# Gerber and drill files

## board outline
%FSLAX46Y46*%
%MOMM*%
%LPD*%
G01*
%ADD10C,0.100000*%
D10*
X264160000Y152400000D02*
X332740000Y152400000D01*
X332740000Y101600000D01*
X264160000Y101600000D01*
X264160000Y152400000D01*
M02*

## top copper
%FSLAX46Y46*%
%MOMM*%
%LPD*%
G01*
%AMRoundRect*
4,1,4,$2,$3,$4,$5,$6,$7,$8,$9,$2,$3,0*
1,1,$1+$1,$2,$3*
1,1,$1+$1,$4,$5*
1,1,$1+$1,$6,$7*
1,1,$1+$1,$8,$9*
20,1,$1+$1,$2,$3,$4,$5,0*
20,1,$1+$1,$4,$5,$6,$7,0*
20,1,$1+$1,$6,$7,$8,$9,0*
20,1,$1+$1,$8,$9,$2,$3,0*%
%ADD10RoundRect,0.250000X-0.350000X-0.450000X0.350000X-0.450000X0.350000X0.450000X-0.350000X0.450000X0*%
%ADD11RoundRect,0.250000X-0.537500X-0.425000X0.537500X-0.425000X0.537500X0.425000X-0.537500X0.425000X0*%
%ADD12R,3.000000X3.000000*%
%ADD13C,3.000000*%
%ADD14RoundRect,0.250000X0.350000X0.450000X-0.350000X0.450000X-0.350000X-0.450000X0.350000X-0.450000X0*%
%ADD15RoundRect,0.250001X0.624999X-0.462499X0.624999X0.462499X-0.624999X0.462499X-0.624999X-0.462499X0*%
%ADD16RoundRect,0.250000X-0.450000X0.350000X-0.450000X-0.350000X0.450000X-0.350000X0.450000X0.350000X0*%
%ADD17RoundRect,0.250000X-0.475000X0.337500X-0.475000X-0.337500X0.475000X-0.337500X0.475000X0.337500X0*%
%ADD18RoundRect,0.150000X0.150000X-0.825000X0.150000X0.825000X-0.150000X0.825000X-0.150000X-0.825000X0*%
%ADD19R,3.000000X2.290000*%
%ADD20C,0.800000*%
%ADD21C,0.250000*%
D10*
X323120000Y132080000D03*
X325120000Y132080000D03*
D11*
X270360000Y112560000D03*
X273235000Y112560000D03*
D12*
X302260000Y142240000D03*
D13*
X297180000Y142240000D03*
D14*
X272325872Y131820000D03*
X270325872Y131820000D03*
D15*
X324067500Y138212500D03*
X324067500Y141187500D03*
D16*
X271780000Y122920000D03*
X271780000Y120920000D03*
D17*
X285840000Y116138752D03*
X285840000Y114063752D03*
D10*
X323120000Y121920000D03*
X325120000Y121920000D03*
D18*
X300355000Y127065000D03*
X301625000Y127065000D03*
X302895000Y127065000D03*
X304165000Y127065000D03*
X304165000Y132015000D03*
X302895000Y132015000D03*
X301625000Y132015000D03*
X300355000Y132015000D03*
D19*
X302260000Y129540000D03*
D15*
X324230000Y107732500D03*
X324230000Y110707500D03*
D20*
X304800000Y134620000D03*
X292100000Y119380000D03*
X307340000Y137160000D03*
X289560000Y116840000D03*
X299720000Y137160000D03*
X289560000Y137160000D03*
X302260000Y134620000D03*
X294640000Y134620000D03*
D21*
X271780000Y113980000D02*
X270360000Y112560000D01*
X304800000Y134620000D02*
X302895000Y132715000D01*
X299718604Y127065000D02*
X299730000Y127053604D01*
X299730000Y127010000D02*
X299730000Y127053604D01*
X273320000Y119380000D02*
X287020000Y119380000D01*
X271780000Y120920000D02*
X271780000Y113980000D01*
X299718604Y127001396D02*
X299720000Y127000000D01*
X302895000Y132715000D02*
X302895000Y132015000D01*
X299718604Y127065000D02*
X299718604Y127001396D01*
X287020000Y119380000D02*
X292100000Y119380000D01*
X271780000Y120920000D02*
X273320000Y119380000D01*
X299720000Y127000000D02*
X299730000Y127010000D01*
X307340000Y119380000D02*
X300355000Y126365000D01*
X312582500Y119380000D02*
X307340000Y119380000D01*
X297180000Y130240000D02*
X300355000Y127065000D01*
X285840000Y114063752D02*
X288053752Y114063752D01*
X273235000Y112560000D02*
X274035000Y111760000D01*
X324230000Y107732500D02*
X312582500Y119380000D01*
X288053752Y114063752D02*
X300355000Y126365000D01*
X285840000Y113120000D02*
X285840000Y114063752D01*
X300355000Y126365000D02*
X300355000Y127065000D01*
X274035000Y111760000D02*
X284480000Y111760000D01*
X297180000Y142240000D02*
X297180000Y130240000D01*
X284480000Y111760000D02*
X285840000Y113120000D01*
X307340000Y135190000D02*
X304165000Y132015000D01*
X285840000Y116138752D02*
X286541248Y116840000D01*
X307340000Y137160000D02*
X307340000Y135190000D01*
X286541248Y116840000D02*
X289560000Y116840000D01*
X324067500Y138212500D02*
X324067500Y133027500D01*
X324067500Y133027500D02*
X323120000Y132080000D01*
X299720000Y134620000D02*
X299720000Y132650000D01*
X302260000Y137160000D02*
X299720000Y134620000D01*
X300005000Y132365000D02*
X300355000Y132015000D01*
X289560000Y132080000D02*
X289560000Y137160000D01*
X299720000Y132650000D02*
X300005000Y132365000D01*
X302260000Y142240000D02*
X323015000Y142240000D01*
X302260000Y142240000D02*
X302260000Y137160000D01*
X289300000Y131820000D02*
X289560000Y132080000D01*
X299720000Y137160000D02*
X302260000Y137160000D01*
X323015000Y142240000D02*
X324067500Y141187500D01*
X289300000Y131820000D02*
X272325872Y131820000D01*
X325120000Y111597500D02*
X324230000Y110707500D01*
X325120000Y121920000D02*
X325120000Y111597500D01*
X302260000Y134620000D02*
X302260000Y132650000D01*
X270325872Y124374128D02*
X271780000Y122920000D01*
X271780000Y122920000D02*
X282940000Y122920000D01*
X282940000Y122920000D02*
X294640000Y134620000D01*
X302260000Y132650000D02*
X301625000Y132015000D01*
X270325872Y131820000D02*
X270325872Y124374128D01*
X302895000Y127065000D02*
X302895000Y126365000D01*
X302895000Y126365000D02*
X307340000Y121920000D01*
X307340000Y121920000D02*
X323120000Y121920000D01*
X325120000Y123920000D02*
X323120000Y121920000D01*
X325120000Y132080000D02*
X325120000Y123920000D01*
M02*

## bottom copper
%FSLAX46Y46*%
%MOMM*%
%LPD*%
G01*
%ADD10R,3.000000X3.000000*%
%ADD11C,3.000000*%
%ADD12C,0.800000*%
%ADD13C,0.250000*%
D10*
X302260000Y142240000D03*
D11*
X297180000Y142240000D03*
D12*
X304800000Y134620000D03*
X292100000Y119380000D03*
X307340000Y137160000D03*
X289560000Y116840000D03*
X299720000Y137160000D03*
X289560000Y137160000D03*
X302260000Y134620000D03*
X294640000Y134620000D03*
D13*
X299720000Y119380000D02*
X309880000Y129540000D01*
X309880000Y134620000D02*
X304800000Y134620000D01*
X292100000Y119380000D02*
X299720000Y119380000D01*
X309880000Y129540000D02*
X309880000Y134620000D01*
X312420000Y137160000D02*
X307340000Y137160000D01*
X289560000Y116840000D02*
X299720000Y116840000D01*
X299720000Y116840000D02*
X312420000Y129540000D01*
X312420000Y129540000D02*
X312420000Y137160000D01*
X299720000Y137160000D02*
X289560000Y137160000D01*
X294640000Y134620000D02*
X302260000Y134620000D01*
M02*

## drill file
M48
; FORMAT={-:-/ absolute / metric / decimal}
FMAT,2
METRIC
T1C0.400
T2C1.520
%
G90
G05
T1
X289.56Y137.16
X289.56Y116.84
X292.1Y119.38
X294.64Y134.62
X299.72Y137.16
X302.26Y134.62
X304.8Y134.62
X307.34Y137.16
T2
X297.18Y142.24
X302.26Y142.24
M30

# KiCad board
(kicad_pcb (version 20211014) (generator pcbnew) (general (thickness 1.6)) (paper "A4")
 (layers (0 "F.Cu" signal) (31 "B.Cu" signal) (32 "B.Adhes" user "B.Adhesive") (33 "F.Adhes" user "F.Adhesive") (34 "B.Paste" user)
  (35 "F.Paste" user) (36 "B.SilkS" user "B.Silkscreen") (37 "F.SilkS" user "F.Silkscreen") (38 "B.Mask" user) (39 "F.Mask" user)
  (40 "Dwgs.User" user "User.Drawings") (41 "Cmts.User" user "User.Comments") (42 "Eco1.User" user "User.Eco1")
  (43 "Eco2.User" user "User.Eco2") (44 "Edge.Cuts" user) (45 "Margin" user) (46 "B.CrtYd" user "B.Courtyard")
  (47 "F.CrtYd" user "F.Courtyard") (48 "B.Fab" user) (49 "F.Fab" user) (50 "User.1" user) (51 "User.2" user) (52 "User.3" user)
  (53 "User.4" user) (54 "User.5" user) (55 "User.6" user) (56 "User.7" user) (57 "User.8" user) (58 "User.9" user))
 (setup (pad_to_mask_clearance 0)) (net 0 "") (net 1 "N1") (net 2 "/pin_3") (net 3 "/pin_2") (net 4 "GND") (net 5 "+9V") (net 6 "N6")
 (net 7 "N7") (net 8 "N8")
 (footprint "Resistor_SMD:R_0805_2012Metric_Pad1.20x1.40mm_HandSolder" (layer "F.Cu") (at 324.12 -132.08)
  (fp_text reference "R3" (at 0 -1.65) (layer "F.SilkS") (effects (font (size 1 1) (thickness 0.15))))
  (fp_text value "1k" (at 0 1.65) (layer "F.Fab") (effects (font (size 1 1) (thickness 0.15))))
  (pad "1" smd roundrect (at -1 0) (size 1.2 1.4) (layers "F.Cu" "F.Paste" "F.Mask") (roundrect_rratio 0.208333) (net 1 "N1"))
  (pad "2" smd roundrect (at 1 0) (size 1.2 1.4) (layers "F.Cu" "F.Paste" "F.Mask") (roundrect_rratio 0.208333) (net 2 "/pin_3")))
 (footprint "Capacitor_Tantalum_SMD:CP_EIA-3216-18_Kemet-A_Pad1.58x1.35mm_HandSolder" (layer "F.Cu") (at 271.7975 -112.56)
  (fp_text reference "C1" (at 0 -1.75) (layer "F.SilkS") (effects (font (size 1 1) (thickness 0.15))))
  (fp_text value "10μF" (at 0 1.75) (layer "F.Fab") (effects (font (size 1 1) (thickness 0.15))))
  (pad "1" smd roundrect (at -1.4375 0) (size 1.575 1.35) (layers "F.Cu" "F.Paste" "F.Mask") (roundrect_rratio 0.185185) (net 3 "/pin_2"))
  (pad "2" smd roundrect (at 1.4375 0) (size 1.575 1.35) (layers "F.Cu" "F.Paste" "F.Mask") (roundrect_rratio 0.185185) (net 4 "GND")))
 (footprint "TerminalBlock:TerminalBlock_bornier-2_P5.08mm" (layer "F.Cu") (at 302.26 -142.24 180)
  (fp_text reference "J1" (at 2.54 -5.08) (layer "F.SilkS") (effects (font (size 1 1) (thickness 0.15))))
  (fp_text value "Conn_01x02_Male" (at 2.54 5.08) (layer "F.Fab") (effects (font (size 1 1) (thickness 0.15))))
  (pad "1" thru_hole rect (at 0 0 180) (size 3 3) (drill 1.52) (layers *.Cu *.Mask) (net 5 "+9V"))
  (pad "2" thru_hole circle (at 5.08 0 180) (size 3 3) (drill 1.52) (layers *.Cu *.Mask) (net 4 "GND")))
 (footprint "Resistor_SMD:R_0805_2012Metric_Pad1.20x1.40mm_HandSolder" (layer "F.Cu") (at 271.325872 -131.82 180)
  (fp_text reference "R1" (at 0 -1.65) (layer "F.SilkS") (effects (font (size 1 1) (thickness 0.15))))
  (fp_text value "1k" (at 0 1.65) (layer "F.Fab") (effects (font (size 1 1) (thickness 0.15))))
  (pad "1" smd roundrect (at -1 0 180) (size 1.2 1.4) (layers "F.Cu" "F.Paste" "F.Mask") (roundrect_rratio 0.208333) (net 5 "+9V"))
  (pad "2" smd roundrect (at 1 0 180) (size 1.2 1.4) (layers "F.Cu" "F.Paste" "F.Mask") (roundrect_rratio 0.208333) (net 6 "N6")))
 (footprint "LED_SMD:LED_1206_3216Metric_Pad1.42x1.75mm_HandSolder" (layer "F.Cu") (at 324.0675 -139.7 90)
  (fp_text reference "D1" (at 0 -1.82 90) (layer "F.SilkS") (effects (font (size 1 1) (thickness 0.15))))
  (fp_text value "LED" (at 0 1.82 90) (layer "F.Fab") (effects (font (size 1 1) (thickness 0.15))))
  (pad "1" smd roundrect (at -1.4875 0 90) (size 1.425 1.75) (layers "F.Cu" "F.Paste" "F.Mask") (roundrect_rratio 0.175439) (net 1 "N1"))
  (pad "2" smd roundrect (at 1.4875 0 90) (size 1.425 1.75) (layers "F.Cu" "F.Paste" "F.Mask") (roundrect_rratio 0.175439) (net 5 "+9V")))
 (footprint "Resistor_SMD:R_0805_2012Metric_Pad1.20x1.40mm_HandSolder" (layer "F.Cu") (at 271.78 -121.92 -90)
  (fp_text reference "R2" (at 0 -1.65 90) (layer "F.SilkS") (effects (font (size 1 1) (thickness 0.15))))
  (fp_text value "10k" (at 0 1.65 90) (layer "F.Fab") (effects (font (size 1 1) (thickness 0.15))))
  (pad "1" smd roundrect (at -1 0 270) (size 1.2 1.4) (layers "F.Cu" "F.Paste" "F.Mask") (roundrect_rratio 0.208333) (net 6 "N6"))
  (pad "2" smd roundrect (at 1 0 270) (size 1.2 1.4) (layers "F.Cu" "F.Paste" "F.Mask") (roundrect_rratio 0.208333) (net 3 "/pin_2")))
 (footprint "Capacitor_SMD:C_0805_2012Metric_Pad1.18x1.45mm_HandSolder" (layer "F.Cu") (at 285.84 -115.101252 -90)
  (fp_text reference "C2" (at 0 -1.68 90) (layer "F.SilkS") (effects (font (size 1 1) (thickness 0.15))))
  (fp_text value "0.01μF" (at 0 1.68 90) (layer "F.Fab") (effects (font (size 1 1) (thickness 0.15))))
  (pad "1" smd roundrect (at -1.0375 0 270) (size 1.175 1.45) (layers "F.Cu" "F.Paste" "F.Mask") (roundrect_rratio 0.212766) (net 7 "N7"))
  (pad "2" smd roundrect (at 1.0375 0 270) (size 1.175 1.45) (layers "F.Cu" "F.Paste" "F.Mask") (roundrect_rratio 0.212766) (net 4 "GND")))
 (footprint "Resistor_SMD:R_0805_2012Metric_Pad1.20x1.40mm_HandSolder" (layer "F.Cu") (at 324.12 -121.92)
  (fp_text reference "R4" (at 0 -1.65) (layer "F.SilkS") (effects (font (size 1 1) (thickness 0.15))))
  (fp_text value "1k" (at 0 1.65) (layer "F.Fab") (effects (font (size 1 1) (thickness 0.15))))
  (pad "1" smd roundrect (at -1 0) (size 1.2 1.4) (layers "F.Cu" "F.Paste" "F.Mask") (roundrect_rratio 0.208333) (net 2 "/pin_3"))
  (pad "2" smd roundrect (at 1 0) (size 1.2 1.4) (layers "F.Cu" "F.Paste" "F.Mask") (roundrect_rratio 0.208333) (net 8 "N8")))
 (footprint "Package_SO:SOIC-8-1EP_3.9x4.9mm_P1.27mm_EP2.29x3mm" (layer "F.Cu") (at 302.26 -129.54 90)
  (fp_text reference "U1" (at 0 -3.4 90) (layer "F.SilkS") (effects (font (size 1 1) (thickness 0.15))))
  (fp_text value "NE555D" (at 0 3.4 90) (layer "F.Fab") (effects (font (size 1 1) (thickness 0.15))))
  (pad "" smd roundrect (at 0.57 -0.75 90) (size 0.92 1.21) (layers "F.Paste") (roundrect_rratio 0.25))
  (pad "" smd roundrect (at 0.57 0.75 90) (size 0.92 1.21) (layers "F.Paste") (roundrect_rratio 0.25))
  (pad "" smd roundrect (at -0.57 -0.75 90) (size 0.92 1.21) (layers "F.Paste") (roundrect_rratio 0.25))
  (pad "" smd roundrect (at -0.57 0.75 90) (size 0.92 1.21) (layers "F.Paste") (roundrect_rratio 0.25))
  (pad "1" smd roundrect (at -2.475 -1.905 90) (size 1.95 0.6) (layers "F.Cu" "F.Paste" "F.Mask") (roundrect_rratio 0.25) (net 4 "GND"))
  (pad "2" smd roundrect (at -2.475 -0.635 90) (size 1.95 0.6) (layers "F.Cu" "F.Paste" "F.Mask") (roundrect_rratio 0.25) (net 3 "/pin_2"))
  (pad "3" smd roundrect (at -2.475 0.635 90) (size 1.95 0.6) (layers "F.Cu" "F.Paste" "F.Mask") (roundrect_rratio 0.25) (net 2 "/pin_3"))
  (pad "4" smd roundrect (at -2.475 1.905 90) (size 1.95 0.6) (layers "F.Cu" "F.Paste" "F.Mask") (roundrect_rratio 0.25) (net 5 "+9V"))
  (pad "5" smd roundrect (at 2.475 1.905 90) (size 1.95 0.6) (layers "F.Cu" "F.Paste" "F.Mask") (roundrect_rratio 0.25) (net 7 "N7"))
  (pad "6" smd roundrect (at 2.475 0.635 90) (size 1.95 0.6) (layers "F.Cu" "F.Paste" "F.Mask") (roundrect_rratio 0.25) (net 3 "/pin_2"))
  (pad "7" smd roundrect (at 2.475 -0.635 90) (size 1.95 0.6) (layers "F.Cu" "F.Paste" "F.Mask") (roundrect_rratio 0.25) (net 6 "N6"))
  (pad "8" smd roundrect (at 2.475 -1.905 90) (size 1.95 0.6) (layers "F.Cu" "F.Paste" "F.Mask") (roundrect_rratio 0.25) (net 5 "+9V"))
  (pad "9" smd rect (at 0 0 90) (size 2.29 3) (layers "F.Cu" "F.Mask")))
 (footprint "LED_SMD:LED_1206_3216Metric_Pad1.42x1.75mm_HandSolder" (layer "F.Cu") (at 324.23 -109.22 90)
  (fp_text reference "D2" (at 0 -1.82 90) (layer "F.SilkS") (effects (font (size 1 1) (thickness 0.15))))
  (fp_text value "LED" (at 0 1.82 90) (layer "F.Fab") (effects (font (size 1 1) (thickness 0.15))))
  (pad "1" smd roundrect (at -1.4875 0 90) (size 1.425 1.75) (layers "F.Cu" "F.Paste" "F.Mask") (roundrect_rratio 0.175439) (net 4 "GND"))
  (pad "2" smd roundrect (at 1.4875 0 90) (size 1.425 1.75) (layers "F.Cu" "F.Paste" "F.Mask") (roundrect_rratio 0.175439) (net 8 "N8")))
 (gr_rect (start 264.16 -152.4) (end 332.74 -101.6) (layer "Edge.Cuts") (width 0.1) (fill none))
 (segment (start 271.78 -113.98) (end 270.36 -112.56) (width 0.25) (layer "F.Cu") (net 3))
 (segment (start 304.8 -134.62) (end 302.895 -132.715) (width 0.25) (layer "F.Cu") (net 3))
 (segment (start 299.718604 -127.065) (end 299.73 -127.053604) (width 0.25) (layer "F.Cu") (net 3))
 (segment (start 299.73 -127.01) (end 299.73 -127.053604) (width 0.25) (layer "F.Cu") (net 3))
 (segment (start 273.32 -119.38) (end 287.02 -119.38) (width 0.25) (layer "F.Cu") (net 3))
 (segment (start 271.78 -120.92) (end 271.78 -113.98) (width 0.25) (layer "F.Cu") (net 3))
 (segment (start 299.718604 -127.001396) (end 299.72 -127) (width 0.25) (layer "F.Cu") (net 3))
 (segment (start 302.895 -132.715) (end 302.895 -132.015) (width 0.25) (layer "F.Cu") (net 3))
 (segment (start 299.718604 -127.065) (end 299.718604 -127.001396) (width 0.25) (layer "F.Cu") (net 3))
 (segment (start 287.02 -119.38) (end 292.1 -119.38) (width 0.25) (layer "F.Cu") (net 3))
 (segment (start 271.78 -120.92) (end 273.32 -119.38) (width 0.25) (layer "F.Cu") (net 3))
 (segment (start 299.72 -127) (end 299.73 -127.01) (width 0.25) (layer "F.Cu") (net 3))
 (via (at 304.8 -134.62) (size 0.8) (drill 0.4) (layers "F.Cu" "B.Cu") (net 3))
 (via (at 292.1 -119.38) (size 0.8) (drill 0.4) (layers "F.Cu" "B.Cu") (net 3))
 (segment (start 299.72 -119.38) (end 309.88 -129.54) (width 0.25) (layer "B.Cu") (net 3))
 (segment (start 309.88 -134.62) (end 304.8 -134.62) (width 0.25) (layer "B.Cu") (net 3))
 (segment (start 292.1 -119.38) (end 299.72 -119.38) (width 0.25) (layer "B.Cu") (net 3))
 (segment (start 309.88 -129.54) (end 309.88 -134.62) (width 0.25) (layer "B.Cu") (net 3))
 (segment (start 307.34 -119.38) (end 300.355 -126.365) (width 0.25) (layer "F.Cu") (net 4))
 (segment (start 312.5825 -119.38) (end 307.34 -119.38) (width 0.25) (layer "F.Cu") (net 4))
 (segment (start 297.18 -130.24) (end 300.355 -127.065) (width 0.25) (layer "F.Cu") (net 4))
 (segment (start 285.84 -114.063752) (end 288.053752 -114.063752) (width 0.25) (layer "F.Cu") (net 4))
 (segment (start 273.235 -112.56) (end 274.035 -111.76) (width 0.25) (layer "F.Cu") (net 4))
 (segment (start 324.23 -107.7325) (end 312.5825 -119.38) (width 0.25) (layer "F.Cu") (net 4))
 (segment (start 288.053752 -114.063752) (end 300.355 -126.365) (width 0.25) (layer "F.Cu") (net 4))
 (segment (start 285.84 -113.12) (end 285.84 -114.063752) (width 0.25) (layer "F.Cu") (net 4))
 (segment (start 300.355 -126.365) (end 300.355 -127.065) (width 0.25) (layer "F.Cu") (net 4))
 (segment (start 274.035 -111.76) (end 284.48 -111.76) (width 0.25) (layer "F.Cu") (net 4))
 (segment (start 297.18 -142.24) (end 297.18 -130.24) (width 0.25) (layer "F.Cu") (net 4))
 (segment (start 284.48 -111.76) (end 285.84 -113.12) (width 0.25) (layer "F.Cu") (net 4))
 (segment (start 307.34 -135.19) (end 304.165 -132.015) (width 0.25) (layer "F.Cu") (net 7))
 (segment (start 285.84 -116.138752) (end 286.541248 -116.84) (width 0.25) (layer "F.Cu") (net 7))
 (segment (start 307.34 -137.16) (end 307.34 -135.19) (width 0.25) (layer "F.Cu") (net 7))
 (segment (start 286.541248 -116.84) (end 289.56 -116.84) (width 0.25) (layer "F.Cu") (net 7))
 (via (at 307.34 -137.16) (size 0.8) (drill 0.4) (layers "F.Cu" "B.Cu") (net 7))
 (via (at 289.56 -116.84) (size 0.8) (drill 0.4) (layers "F.Cu" "B.Cu") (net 7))
 (segment (start 312.42 -137.16) (end 307.34 -137.16) (width 0.25) (layer "B.Cu") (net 7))
 (segment (start 289.56 -116.84) (end 299.72 -116.84) (width 0.25) (layer "B.Cu") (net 7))
 (segment (start 299.72 -116.84) (end 312.42 -129.54) (width 0.25) (layer "B.Cu") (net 7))
 (segment (start 312.42 -129.54) (end 312.42 -137.16) (width 0.25) (layer "B.Cu") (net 7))
 (segment (start 324.0675 -138.2125) (end 324.0675 -133.0275) (width 0.25) (layer "F.Cu") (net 1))
 (segment (start 324.0675 -133.0275) (end 323.12 -132.08) (width 0.25) (layer "F.Cu") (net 1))
 (segment (start 299.72 -134.62) (end 299.72 -132.65) (width 0.25) (layer "F.Cu") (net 5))
 (segment (start 302.26 -137.16) (end 299.72 -134.62) (width 0.25) (layer "F.Cu") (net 5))
 (segment (start 300.005 -132.365) (end 300.355 -132.015) (width 0.25) (layer "F.Cu") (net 5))
 (segment (start 289.56 -132.08) (end 289.56 -137.16) (width 0.25) (layer "F.Cu") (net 5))
 (segment (start 299.72 -132.65) (end 300.005 -132.365) (width 0.25) (layer "F.Cu") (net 5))
 (segment (start 302.26 -142.24) (end 323.015 -142.24) (width 0.25) (layer "F.Cu") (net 5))
 (segment (start 302.26 -142.24) (end 302.26 -137.16) (width 0.25) (layer "F.Cu") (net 5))
 (segment (start 289.3 -131.82) (end 289.56 -132.08) (width 0.25) (layer "F.Cu") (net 5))
 (segment (start 299.72 -137.16) (end 302.26 -137.16) (width 0.25) (layer "F.Cu") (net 5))
 (segment (start 323.015 -142.24) (end 324.0675 -141.1875) (width 0.25) (layer "F.Cu") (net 5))
 (segment (start 289.3 -131.82) (end 272.325872 -131.82) (width 0.25) (layer "F.Cu") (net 5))
 (via (at 299.72 -137.16) (size 0.8) (drill 0.4) (layers "F.Cu" "B.Cu") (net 5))
 (via (at 289.56 -137.16) (size 0.8) (drill 0.4) (layers "F.Cu" "B.Cu") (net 5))
 (segment (start 299.72 -137.16) (end 289.56 -137.16) (width 0.25) (layer "B.Cu") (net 5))
 (segment (start 325.12 -111.5975) (end 324.23 -110.7075) (width 0.25) (layer "F.Cu") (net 8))
 (segment (start 325.12 -121.92) (end 325.12 -111.5975) (width 0.25) (layer "F.Cu") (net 8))
 (segment (start 302.26 -134.62) (end 302.26 -132.65) (width 0.25) (layer "F.Cu") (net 6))
 (segment (start 270.325872 -124.374128) (end 271.78 -122.92) (width 0.25) (layer "F.Cu") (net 6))
 (segment (start 271.78 -122.92) (end 282.94 -122.92) (width 0.25) (layer "F.Cu") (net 6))
 (segment (start 282.94 -122.92) (end 294.64 -134.62) (width 0.25) (layer "F.Cu") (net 6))
 (segment (start 302.26 -132.65) (end 301.625 -132.015) (width 0.25) (layer "F.Cu") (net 6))
 (segment (start 270.325872 -131.82) (end 270.325872 -124.374128) (width 0.25) (layer "F.Cu") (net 6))
 (via (at 302.26 -134.62) (size 0.8) (drill 0.4) (layers "F.Cu" "B.Cu") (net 6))
 (via (at 294.64 -134.62) (size 0.8) (drill 0.4) (layers "F.Cu" "B.Cu") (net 6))
 (segment (start 294.64 -134.62) (end 302.26 -134.62) (width 0.25) (layer "B.Cu") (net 6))
 (segment (start 302.895 -127.065) (end 302.895 -126.365) (width 0.25) (layer "F.Cu") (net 2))
 (segment (start 302.895 -126.365) (end 307.34 -121.92) (width 0.25) (layer "F.Cu") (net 2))
 (segment (start 307.34 -121.92) (end 323.12 -121.92) (width 0.25) (layer "F.Cu") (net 2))
 (segment (start 325.12 -123.92) (end 323.12 -121.92) (width 0.25) (layer "F.Cu") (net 2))
 (segment (start 325.12 -132.08) (end 325.12 -123.92) (width 0.25) (layer "F.Cu") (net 2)))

